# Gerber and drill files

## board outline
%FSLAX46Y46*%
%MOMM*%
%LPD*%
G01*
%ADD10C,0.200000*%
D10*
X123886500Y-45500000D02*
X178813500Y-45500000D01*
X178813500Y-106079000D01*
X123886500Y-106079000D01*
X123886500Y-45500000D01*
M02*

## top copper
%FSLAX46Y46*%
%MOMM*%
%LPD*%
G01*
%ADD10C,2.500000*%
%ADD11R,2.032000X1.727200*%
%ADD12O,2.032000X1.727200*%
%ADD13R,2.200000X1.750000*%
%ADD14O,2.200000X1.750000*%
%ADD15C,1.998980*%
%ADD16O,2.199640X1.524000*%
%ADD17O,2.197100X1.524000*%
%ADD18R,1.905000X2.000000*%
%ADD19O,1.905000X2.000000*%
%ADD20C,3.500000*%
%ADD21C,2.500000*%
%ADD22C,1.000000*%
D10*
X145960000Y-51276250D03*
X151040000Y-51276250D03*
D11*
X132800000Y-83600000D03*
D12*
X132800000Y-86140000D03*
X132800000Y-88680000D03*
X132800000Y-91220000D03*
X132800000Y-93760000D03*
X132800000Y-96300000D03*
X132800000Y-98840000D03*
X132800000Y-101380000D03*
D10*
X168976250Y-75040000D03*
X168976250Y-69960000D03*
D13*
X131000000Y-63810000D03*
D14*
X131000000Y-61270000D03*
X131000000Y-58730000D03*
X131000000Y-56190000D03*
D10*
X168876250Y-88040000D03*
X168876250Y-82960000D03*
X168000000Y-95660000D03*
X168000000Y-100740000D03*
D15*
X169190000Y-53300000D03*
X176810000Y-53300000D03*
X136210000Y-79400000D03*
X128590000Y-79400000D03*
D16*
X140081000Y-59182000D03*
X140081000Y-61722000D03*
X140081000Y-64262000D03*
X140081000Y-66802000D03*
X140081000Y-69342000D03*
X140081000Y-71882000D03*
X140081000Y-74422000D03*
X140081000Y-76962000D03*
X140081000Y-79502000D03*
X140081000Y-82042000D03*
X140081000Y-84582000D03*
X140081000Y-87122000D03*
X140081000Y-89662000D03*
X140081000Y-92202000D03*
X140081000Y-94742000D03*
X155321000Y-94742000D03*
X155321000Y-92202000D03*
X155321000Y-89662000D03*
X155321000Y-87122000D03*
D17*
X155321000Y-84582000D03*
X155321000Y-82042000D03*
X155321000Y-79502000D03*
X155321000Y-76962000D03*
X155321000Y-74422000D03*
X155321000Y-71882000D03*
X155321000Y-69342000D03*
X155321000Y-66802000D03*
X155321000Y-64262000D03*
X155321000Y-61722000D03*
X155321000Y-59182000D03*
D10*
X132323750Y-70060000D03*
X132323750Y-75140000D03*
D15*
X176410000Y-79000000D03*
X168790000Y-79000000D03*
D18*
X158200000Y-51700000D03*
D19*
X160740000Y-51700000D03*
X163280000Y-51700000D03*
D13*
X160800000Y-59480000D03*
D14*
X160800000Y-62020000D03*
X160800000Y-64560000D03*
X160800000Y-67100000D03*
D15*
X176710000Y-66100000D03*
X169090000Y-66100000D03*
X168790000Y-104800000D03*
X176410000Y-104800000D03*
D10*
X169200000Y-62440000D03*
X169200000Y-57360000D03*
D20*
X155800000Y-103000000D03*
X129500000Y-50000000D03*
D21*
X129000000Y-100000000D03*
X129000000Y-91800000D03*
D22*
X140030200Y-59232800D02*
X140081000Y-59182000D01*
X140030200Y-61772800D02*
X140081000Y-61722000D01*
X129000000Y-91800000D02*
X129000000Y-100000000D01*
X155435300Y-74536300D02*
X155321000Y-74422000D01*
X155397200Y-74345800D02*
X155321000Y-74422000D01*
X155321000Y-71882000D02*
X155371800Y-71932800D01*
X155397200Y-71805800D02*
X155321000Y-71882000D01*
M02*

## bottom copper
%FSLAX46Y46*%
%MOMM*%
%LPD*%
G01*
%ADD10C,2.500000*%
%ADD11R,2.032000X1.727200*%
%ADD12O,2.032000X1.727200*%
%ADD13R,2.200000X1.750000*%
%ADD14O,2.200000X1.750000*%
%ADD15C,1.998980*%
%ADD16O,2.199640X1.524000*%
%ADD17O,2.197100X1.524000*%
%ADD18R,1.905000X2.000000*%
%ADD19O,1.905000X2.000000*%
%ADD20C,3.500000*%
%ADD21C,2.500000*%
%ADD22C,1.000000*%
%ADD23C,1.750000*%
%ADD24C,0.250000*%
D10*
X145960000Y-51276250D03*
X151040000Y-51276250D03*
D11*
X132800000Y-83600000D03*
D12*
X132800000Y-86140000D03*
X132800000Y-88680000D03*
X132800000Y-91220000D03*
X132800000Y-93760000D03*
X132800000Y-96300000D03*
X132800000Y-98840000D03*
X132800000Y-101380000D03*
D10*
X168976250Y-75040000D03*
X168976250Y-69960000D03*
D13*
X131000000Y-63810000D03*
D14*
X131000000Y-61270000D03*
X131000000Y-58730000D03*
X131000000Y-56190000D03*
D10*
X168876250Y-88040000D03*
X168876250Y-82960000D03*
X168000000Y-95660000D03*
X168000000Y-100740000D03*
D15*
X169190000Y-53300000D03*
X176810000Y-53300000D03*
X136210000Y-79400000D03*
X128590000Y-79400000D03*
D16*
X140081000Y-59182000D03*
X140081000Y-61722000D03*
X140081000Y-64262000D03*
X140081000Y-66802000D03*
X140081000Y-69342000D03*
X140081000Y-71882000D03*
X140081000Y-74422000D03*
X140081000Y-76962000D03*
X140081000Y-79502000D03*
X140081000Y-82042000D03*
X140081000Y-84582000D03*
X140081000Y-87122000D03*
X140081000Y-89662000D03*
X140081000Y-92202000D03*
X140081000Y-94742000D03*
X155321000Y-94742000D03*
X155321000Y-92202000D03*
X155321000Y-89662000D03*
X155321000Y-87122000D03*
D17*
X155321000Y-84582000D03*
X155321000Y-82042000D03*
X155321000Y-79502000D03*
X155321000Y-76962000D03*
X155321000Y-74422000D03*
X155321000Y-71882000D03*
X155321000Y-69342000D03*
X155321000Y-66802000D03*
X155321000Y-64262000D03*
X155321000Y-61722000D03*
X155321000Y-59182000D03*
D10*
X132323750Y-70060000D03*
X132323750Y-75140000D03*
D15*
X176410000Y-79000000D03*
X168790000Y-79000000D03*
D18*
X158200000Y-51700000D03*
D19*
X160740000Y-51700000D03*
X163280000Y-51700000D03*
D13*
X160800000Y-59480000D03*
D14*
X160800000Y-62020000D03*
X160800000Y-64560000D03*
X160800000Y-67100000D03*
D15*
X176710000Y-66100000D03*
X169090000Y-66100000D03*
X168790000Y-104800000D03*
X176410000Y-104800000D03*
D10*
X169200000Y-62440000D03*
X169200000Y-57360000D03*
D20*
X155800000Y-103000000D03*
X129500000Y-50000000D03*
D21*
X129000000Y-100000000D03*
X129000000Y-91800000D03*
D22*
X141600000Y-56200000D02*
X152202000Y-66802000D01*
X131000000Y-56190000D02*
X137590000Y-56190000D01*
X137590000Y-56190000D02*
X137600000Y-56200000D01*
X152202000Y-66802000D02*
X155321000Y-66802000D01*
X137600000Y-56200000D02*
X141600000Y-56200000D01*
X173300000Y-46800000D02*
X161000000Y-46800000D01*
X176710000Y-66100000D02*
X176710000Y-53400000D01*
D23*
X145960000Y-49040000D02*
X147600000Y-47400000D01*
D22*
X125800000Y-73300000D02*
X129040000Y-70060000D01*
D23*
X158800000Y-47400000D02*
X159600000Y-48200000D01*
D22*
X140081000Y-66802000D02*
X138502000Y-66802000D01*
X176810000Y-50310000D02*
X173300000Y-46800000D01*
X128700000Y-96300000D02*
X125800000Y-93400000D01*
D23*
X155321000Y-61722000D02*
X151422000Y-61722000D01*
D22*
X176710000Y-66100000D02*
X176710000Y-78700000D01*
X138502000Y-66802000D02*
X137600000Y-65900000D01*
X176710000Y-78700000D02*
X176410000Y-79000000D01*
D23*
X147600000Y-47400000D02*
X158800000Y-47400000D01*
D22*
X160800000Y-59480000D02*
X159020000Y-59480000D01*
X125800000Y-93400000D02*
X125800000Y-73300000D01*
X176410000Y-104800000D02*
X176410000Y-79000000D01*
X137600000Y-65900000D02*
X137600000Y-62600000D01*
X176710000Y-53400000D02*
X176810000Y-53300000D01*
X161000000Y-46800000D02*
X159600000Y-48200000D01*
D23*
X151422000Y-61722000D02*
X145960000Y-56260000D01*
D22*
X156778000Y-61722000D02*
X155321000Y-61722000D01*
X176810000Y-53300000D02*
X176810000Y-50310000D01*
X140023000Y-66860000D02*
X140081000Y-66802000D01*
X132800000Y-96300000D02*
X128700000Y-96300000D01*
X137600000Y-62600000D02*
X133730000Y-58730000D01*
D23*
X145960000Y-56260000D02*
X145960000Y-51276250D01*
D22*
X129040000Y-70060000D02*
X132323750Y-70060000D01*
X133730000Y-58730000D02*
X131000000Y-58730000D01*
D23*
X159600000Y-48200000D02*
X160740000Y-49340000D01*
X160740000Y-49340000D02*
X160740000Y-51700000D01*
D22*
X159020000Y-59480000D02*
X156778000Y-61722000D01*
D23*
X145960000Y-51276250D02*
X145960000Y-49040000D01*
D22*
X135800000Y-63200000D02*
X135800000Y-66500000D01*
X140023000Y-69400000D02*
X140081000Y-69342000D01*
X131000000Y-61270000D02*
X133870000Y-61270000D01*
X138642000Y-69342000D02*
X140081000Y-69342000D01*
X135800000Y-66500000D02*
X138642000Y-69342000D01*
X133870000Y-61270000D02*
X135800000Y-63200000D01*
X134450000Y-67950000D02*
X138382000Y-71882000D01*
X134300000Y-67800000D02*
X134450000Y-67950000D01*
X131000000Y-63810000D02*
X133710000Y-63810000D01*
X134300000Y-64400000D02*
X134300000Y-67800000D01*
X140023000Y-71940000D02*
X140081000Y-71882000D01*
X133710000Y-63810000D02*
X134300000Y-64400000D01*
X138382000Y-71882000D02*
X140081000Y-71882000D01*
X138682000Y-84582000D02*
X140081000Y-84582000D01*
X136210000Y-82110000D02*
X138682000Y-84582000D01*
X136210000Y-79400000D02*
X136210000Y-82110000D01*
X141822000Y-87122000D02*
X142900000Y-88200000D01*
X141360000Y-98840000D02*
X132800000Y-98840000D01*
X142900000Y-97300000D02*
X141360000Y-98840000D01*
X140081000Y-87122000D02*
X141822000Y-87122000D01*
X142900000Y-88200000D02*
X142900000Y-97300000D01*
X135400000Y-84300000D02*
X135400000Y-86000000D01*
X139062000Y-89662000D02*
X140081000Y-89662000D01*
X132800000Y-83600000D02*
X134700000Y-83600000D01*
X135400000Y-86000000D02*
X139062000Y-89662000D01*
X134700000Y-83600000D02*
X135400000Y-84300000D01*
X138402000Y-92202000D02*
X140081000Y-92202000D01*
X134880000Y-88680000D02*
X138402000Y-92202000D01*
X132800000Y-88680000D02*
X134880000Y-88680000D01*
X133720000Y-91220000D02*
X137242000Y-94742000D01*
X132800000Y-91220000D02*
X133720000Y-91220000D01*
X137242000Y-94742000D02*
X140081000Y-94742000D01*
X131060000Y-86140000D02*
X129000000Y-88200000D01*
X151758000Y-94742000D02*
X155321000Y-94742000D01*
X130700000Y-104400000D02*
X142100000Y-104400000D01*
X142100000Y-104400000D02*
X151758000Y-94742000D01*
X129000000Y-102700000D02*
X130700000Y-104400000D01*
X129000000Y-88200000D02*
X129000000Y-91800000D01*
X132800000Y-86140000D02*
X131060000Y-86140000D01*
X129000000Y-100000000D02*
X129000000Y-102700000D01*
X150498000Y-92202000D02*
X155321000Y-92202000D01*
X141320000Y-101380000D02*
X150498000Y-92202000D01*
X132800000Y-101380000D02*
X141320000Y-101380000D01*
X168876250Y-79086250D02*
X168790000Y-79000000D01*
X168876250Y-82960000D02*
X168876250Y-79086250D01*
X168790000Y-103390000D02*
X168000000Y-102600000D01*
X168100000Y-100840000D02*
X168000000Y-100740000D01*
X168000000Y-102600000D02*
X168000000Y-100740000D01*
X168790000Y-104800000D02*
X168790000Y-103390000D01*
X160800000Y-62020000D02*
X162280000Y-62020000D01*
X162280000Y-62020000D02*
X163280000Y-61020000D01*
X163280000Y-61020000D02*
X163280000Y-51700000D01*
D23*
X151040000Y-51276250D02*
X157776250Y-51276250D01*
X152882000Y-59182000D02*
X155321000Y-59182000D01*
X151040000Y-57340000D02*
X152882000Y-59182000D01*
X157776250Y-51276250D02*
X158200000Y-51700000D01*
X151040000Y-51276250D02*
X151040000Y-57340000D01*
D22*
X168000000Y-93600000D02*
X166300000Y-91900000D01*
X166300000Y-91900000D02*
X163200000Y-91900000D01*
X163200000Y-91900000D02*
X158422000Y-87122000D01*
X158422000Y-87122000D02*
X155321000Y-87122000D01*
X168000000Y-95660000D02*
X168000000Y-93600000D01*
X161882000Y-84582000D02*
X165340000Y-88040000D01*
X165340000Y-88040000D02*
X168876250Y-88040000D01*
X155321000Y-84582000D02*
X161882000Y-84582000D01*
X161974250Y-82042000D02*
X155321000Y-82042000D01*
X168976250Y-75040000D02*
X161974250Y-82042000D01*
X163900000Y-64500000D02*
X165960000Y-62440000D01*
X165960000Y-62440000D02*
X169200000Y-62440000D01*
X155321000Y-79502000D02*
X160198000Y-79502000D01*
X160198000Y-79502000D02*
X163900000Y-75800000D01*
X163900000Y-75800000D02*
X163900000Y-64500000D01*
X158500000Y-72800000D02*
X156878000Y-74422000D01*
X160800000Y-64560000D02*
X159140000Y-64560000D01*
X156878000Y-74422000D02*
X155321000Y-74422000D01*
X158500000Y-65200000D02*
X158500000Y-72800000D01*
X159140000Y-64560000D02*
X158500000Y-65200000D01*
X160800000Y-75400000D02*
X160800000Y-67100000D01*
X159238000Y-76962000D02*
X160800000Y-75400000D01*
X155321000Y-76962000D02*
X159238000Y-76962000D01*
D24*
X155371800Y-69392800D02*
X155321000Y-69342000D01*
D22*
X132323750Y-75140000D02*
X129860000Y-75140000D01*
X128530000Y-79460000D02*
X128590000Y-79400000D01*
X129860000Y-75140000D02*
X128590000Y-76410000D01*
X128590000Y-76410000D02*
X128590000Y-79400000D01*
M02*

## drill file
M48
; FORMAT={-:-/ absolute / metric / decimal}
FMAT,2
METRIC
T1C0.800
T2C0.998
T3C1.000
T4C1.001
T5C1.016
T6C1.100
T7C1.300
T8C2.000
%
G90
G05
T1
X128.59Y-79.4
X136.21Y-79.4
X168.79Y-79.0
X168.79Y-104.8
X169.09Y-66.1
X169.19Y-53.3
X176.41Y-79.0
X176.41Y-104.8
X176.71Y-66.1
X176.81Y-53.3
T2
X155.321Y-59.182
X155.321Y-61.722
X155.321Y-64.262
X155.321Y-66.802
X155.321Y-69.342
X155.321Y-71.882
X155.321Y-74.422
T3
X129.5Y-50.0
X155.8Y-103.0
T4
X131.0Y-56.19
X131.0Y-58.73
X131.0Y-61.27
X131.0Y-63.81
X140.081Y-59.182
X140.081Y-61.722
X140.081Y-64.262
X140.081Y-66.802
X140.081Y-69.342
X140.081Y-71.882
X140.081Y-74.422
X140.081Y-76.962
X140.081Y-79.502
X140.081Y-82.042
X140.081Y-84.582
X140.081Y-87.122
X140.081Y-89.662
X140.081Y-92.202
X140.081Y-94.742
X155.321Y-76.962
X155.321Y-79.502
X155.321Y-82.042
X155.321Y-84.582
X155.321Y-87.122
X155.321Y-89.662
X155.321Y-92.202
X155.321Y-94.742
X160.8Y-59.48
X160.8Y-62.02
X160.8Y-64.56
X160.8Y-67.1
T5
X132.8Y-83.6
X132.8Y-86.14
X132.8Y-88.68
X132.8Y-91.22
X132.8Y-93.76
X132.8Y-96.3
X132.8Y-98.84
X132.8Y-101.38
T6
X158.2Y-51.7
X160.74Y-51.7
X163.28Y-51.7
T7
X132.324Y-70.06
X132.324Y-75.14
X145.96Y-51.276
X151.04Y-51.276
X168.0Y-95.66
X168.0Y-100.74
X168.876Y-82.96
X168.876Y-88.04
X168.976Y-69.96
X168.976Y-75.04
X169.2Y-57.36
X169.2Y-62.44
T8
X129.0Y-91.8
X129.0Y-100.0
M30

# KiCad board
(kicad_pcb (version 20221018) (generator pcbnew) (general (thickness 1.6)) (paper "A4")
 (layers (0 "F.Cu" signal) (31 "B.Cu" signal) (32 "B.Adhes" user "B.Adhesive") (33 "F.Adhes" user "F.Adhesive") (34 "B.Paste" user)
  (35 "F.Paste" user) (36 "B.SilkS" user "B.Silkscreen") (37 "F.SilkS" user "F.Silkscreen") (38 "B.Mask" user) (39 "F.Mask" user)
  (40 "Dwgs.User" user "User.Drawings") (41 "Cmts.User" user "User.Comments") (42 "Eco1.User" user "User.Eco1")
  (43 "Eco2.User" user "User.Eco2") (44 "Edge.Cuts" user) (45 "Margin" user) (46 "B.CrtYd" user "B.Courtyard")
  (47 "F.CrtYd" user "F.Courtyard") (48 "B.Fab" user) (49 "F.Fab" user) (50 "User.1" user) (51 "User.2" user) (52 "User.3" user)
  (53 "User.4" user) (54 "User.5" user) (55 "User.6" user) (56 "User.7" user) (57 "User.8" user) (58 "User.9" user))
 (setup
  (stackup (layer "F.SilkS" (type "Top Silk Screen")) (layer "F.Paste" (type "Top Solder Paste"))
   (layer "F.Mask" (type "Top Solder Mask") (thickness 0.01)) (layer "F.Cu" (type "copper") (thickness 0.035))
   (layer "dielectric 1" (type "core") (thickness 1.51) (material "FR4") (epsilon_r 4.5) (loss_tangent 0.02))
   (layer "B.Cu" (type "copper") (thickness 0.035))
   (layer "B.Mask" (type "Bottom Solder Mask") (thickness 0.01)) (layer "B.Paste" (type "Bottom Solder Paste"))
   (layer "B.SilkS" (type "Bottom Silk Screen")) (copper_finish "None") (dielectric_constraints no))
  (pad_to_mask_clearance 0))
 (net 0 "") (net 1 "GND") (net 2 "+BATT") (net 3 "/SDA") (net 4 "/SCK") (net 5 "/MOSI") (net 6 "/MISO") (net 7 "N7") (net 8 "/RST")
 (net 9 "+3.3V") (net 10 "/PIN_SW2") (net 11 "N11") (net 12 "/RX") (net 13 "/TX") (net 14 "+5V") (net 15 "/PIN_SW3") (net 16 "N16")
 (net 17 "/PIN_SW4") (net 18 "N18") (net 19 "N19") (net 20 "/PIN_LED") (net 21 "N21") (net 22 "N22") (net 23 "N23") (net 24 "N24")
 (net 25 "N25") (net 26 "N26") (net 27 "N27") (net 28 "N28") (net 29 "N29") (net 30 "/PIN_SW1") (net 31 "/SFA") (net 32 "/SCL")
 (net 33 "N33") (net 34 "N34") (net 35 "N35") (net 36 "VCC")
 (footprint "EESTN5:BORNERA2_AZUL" (layer "F.Cu") (at 148.5 51.27625)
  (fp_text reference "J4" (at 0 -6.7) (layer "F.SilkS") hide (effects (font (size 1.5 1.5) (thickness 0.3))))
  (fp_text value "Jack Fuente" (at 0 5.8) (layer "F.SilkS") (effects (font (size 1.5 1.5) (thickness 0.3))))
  (pad "1" thru_hole circle (at -2.54 0) (size 2.5 2.5) (drill 1.3) (layers "*.Cu" "*.Mask" "F.SilkS") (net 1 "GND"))
  (pad "2" thru_hole circle (at 2.54 0) (size 2.5 2.5) (drill 1.3) (layers "*.Cu" "*.Mask" "F.SilkS") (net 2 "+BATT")))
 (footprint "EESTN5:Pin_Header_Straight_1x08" (layer "F.Cu") (at 132.8 83.6)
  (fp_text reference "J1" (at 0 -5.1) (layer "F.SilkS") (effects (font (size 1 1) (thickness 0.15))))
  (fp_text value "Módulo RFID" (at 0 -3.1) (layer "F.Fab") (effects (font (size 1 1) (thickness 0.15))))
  (pad "1" thru_hole rect (at 0 0) (size 2.032 1.7272) (drill 1.016) (layers "*.Cu" "*.Mask" "F.SilkS") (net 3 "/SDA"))
  (pad "2" thru_hole oval (at 0 2.54) (size 2.032 1.7272) (drill 1.016) (layers "*.Cu" "*.Mask" "F.SilkS") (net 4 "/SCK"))
  (pad "3" thru_hole oval (at 0 5.08) (size 2.032 1.7272) (drill 1.016) (layers "*.Cu" "*.Mask" "F.SilkS") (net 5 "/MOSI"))
  (pad "4" thru_hole oval (at 0 7.62) (size 2.032 1.7272) (drill 1.016) (layers "*.Cu" "*.Mask" "F.SilkS") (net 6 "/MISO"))
  (pad "5" thru_hole oval (at 0 10.16) (size 2.032 1.7272) (drill 1.016) (layers "*.Cu" "*.Mask" "F.SilkS") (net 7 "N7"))
  (pad "6" thru_hole oval (at 0 12.7) (size 2.032 1.7272) (drill 1.016) (layers "*.Cu" "*.Mask" "F.SilkS") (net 1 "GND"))
  (pad "7" thru_hole oval (at 0 15.24) (size 2.032 1.7272) (drill 1.016) (layers "*.Cu" "*.Mask" "F.SilkS") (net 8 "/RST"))
  (pad "8" thru_hole oval (at 0 17.78) (size 2.032 1.7272) (drill 1.016) (layers "*.Cu" "*.Mask" "F.SilkS") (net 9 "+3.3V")))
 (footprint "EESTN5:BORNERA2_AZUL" (layer "F.Cu") (at 168.97625 72.5 90)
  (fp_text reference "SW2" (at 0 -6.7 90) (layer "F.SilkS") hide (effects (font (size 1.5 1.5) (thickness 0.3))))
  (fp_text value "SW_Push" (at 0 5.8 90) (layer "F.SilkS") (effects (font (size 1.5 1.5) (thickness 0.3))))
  (pad "1" thru_hole circle (at -2.54 0 90) (size 2.5 2.5) (drill 1.3) (layers "*.Cu" "*.Mask" "F.SilkS") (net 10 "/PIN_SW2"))
  (pad "2" thru_hole circle (at 2.54 0 90) (size 2.5 2.5) (drill 1.3) (layers "*.Cu" "*.Mask" "F.SilkS") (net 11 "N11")))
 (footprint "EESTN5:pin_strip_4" (layer "F.Cu") (at 131 60 90)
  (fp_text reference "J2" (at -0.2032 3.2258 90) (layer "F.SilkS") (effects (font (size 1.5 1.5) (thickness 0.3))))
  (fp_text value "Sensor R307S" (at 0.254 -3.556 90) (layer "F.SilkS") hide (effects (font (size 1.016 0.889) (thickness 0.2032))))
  (pad "1" thru_hole rect (at -3.81 0 90) (size 1.75 2.2) (drill 1.00076) (layers "*.Cu" "*.Mask" "F.SilkS") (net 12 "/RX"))
  (pad "2" thru_hole oval (at -1.27 0 90) (size 1.75 2.2) (drill 1.00076) (layers "*.Cu" "*.Mask" "F.SilkS") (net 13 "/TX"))
  (pad "3" thru_hole oval (at 1.27 0 90) (size 1.75 2.2) (drill 1.00076) (layers "*.Cu" "*.Mask" "F.SilkS") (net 1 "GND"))
  (pad "4" thru_hole oval (at 3.81 0 90) (size 1.75 2.2) (drill 1.00076) (layers "*.Cu" "*.Mask" "F.SilkS") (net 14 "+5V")))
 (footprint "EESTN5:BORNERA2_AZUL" (layer "F.Cu") (at 168.87625 85.5 90)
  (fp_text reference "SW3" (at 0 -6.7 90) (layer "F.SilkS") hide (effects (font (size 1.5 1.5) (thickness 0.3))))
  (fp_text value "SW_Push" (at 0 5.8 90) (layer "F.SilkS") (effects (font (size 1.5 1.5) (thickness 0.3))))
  (pad "1" thru_hole circle (at -2.54 0 90) (size 2.5 2.5) (drill 1.3) (layers "*.Cu" "*.Mask" "F.SilkS") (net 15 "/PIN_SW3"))
  (pad "2" thru_hole circle (at 2.54 0 90) (size 2.5 2.5) (drill 1.3) (layers "*.Cu" "*.Mask" "F.SilkS") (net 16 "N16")))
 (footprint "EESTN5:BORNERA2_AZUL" (layer "F.Cu") (at 168 98.2 -90)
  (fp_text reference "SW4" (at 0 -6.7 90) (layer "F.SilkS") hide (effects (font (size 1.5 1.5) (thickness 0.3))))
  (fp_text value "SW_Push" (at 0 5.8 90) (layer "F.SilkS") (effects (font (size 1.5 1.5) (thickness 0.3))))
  (pad "1" thru_hole circle (at -2.54 0 270) (size 2.5 2.5) (drill 1.3) (layers "*.Cu" "*.Mask" "F.SilkS") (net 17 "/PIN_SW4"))
  (pad "2" thru_hole circle (at 2.54 0 270) (size 2.5 2.5) (drill 1.3) (layers "*.Cu" "*.Mask" "F.SilkS") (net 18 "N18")))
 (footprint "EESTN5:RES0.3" (layer "F.Cu") (at 173 53.3)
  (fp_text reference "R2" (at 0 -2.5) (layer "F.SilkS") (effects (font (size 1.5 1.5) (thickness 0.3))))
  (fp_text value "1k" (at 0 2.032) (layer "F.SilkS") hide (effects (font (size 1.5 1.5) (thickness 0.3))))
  (pad "1" thru_hole circle (at -3.81 0) (size 1.99898 1.99898) (drill 0.8001) (layers "*.Cu" "*.Mask" "F.SilkS") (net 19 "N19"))
  (pad "2" thru_hole circle (at 3.81 0) (size 1.99898 1.99898) (drill 0.8001) (layers "*.Cu" "*.Mask" "F.SilkS") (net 1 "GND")))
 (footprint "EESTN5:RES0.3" (layer "F.Cu") (at 132.4 79.4 180)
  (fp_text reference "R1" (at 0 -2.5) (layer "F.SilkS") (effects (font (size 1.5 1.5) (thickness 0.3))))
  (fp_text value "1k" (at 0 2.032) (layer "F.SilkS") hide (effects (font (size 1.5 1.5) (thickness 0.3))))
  (pad "1" thru_hole circle (at -3.81 0 180) (size 1.99898 1.99898) (drill 0.8001) (layers "*.Cu" "*.Mask" "F.SilkS") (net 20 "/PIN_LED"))
  (pad "2" thru_hole circle (at 3.81 0 180) (size 1.99898 1.99898) (drill 0.8001) (layers "*.Cu" "*.Mask" "F.SilkS") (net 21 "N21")))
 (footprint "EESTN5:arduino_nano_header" (layer "F.Cu") (at 147.701 76.962 -90)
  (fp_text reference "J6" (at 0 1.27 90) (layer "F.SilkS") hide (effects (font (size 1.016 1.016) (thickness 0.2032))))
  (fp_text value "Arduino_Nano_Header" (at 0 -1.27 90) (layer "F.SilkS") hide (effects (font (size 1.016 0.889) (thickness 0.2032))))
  (pad "1" thru_hole oval (at -17.78 7.62 270) (size 1.524 2.19964) (drill 1.00076) (layers "*.Cu" "*.Mask" "F.SilkS") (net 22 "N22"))
  (pad "2" thru_hole oval (at -15.24 7.62 270) (size 1.524 2.19964) (drill 1.00076) (layers "*.Cu" "*.Mask" "F.SilkS") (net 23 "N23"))
  (pad "3" thru_hole oval (at -12.7 7.62 270) (size 1.524 2.19964) (drill 1.00076) (layers "*.Cu" "*.Mask" "F.SilkS") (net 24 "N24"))
  (pad "4" thru_hole oval (at -10.16 7.62 270) (size 1.524 2.19964) (drill 1.00076) (layers "*.Cu" "*.Mask" "F.SilkS") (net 1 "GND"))
  (pad "5" thru_hole oval (at -7.62 7.62 270) (size 1.524 2.19964) (drill 1.00076) (layers "*.Cu" "*.Mask" "F.SilkS") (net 13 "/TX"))
  (pad "6" thru_hole oval (at -5.08 7.62 270) (size 1.524 2.19964) (drill 1.00076) (layers "*.Cu" "*.Mask" "F.SilkS") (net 12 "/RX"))
  (pad "7" thru_hole oval (at -2.54 7.62 270) (size 1.524 2.19964) (drill 1.00076) (layers "*.Cu" "*.Mask" "F.SilkS") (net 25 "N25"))
  (pad "8" thru_hole oval (at 0 7.62 270) (size 1.524 2.19964) (drill 1.00076) (layers "*.Cu" "*.Mask" "F.SilkS") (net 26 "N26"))
  (pad "9" thru_hole oval (at 2.54 7.62 270) (size 1.524 2.19964) (drill 1.00076) (layers "*.Cu" "*.Mask" "F.SilkS") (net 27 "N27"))
  (pad "10" thru_hole oval (at 5.08 7.62 270) (size 1.524 2.19964) (drill 1.00076) (layers "*.Cu" "*.Mask" "F.SilkS") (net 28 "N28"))
  (pad "11" thru_hole oval (at 7.62 7.62 270) (size 1.524 2.19964) (drill 1.00076) (layers "*.Cu" "*.Mask" "F.SilkS") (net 20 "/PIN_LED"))
  (pad "12" thru_hole oval (at 10.16 7.62 270) (size 1.524 2.19964) (drill 1.00076) (layers "*.Cu" "*.Mask" "F.SilkS") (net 8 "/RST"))
  (pad "13" thru_hole oval (at 12.7 7.62 270) (size 1.524 2.19964) (drill 1.00076) (layers "*.Cu" "*.Mask" "F.SilkS") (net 3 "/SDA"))
  (pad "14" thru_hole oval (at 15.24 7.62 270) (size 1.524 2.19964) (drill 1.00076) (layers "*.Cu" "*.Mask" "F.SilkS") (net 5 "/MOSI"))
  (pad "15" thru_hole oval (at 17.78 7.62 270) (size 1.524 2.19964) (drill 1.00076) (layers "*.Cu" "*.Mask" "F.SilkS") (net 6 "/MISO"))
  (pad "16" thru_hole oval (at 17.78 -7.62 270) (size 1.524 2.19964) (drill 1.00076) (layers "*.Cu" "*.Mask" "F.SilkS") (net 4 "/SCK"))
  (pad "17" thru_hole oval (at 15.24 -7.62 270) (size 1.524 2.19964) (drill 1.00076) (layers "*.Cu" "*.Mask" "F.SilkS") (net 9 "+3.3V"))
  (pad "18" thru_hole oval (at 12.7 -7.62 270) (size 1.524 2.19964) (drill 1.00076) (layers "*.Cu" "*.Mask" "F.SilkS") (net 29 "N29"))
  (pad "19" thru_hole oval (at 10.16 -7.62 270) (size 1.524 2.19964) (drill 1.00076) (layers "*.Cu" "*.Mask" "F.SilkS") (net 17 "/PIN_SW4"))
  (pad "20" thru_hole oval (at 7.62 -7.62 270) (size 1.524 2.1971) (drill 1.00076) (layers "*.Cu" "*.Mask" "F.SilkS") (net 15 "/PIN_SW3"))
  (pad "21" thru_hole oval (at 5.08 -7.62 270) (size 1.524 2.1971) (drill 1.00076) (layers "*.Cu" "*.Mask" "F.SilkS") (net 10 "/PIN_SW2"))
  (pad "22" thru_hole oval (at 2.54 -7.62 270) (size 1.524 2.1971) (drill 1.00076) (layers "*.Cu" "*.Mask" "F.SilkS") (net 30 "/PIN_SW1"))
  (pad "23" thru_hole oval (at 0 -7.62 270) (size 1.524 2.1971) (drill 1.00076) (layers "*.Cu" "*.Mask" "F.SilkS") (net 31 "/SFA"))
  (pad "24" thru_hole oval (at -2.54 -7.62 270) (size 1.524 2.1971) (drill 0.99822) (layers "*.Cu" "*.Mask" "F.SilkS") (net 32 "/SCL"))
  (pad "25" thru_hole oval (at -5.08 -7.62 270) (size 1.524 2.1971) (drill 0.99822) (layers "*.Cu" "*.Mask" "F.SilkS") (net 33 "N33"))
  (pad "26" thru_hole oval (at -7.62 -7.62 270) (size 1.524 2.1971) (drill 0.99822) (layers "*.Cu" "*.Mask" "F.SilkS") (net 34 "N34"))
  (pad "27" thru_hole oval (at -10.16 -7.62 270) (size 1.524 2.1971) (drill 0.99822) (layers "*.Cu" "*.Mask" "F.SilkS") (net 14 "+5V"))
  (pad "28" thru_hole oval (at -12.7 -7.62 270) (size 1.524 2.1971) (drill 0.99822) (layers "*.Cu" "*.Mask" "F.SilkS") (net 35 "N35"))
  (pad "29" thru_hole oval (at -15.24 -7.62 270) (size 1.524 2.1971) (drill 0.99822) (layers "*.Cu" "*.Mask" "F.SilkS") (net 1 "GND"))
  (pad "30" thru_hole oval (at -17.78 -7.62 270) (size 1.524 2.1971) (drill 0.99822) (layers "*.Cu" "*.Mask" "F.SilkS") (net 2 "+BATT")))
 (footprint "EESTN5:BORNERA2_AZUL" (layer "F.Cu") (at 132.32375 72.6 -90)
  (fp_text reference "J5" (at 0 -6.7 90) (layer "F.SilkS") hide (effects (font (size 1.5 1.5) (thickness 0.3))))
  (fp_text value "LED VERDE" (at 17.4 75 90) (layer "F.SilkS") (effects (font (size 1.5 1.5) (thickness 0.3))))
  (pad "1" thru_hole circle (at -2.54 0 270) (size 2.5 2.5) (drill 1.3) (layers "*.Cu" "*.Mask" "F.SilkS") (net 1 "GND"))
  (pad "2" thru_hole circle (at 2.54 0 270) (size 2.5 2.5) (drill 1.3) (layers "*.Cu" "*.Mask" "F.SilkS") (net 21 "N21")))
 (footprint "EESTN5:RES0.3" (layer "F.Cu") (at 172.6 79 180)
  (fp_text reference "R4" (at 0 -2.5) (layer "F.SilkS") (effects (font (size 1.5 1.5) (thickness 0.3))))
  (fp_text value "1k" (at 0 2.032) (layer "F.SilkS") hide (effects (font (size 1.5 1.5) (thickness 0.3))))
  (pad "1" thru_hole circle (at -3.81 0 180) (size 1.99898 1.99898) (drill 0.8001) (layers "*.Cu" "*.Mask" "F.SilkS") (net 1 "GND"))
  (pad "2" thru_hole circle (at 3.81 0 180) (size 1.99898 1.99898) (drill 0.8001) (layers "*.Cu" "*.Mask" "F.SilkS") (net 16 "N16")))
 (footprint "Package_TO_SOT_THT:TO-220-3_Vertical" (layer "F.Cu") (at 158.2 51.7)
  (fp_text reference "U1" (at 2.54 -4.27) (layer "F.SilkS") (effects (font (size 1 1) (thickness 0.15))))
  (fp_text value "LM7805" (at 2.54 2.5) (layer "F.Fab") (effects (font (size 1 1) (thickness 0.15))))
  (pad "1" thru_hole rect (at 0 0) (size 1.905 2) (drill 1.1) (layers "*.Cu" "*.Mask") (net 2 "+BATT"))
  (pad "2" thru_hole oval (at 2.54 0) (size 1.905 2) (drill 1.1) (layers "*.Cu" "*.Mask") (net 1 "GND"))
  (pad "3" thru_hole oval (at 5.08 0) (size 1.905 2) (drill 1.1) (layers "*.Cu" "*.Mask") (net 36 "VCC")))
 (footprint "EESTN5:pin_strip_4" (layer "F.Cu") (at 160.8 63.29 -90)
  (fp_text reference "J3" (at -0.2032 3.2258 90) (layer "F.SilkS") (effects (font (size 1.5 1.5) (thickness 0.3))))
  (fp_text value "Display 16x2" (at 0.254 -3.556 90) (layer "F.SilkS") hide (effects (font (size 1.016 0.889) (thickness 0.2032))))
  (pad "1" thru_hole rect (at -3.81 0 270) (size 1.75 2.2) (drill 1.00076) (layers "*.Cu" "*.Mask" "F.SilkS") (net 1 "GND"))
  (pad "2" thru_hole oval (at -1.27 0 270) (size 1.75 2.2) (drill 1.00076) (layers "*.Cu" "*.Mask" "F.SilkS") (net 36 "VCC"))
  (pad "3" thru_hole oval (at 1.27 0 270) (size 1.75 2.2) (drill 1.00076) (layers "*.Cu" "*.Mask" "F.SilkS") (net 32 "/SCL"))
  (pad "4" thru_hole oval (at 3.81 0 270) (size 1.75 2.2) (drill 1.00076) (layers "*.Cu" "*.Mask" "F.SilkS") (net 31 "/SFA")))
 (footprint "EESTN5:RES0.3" (layer "F.Cu") (at 172.9 66.1 180)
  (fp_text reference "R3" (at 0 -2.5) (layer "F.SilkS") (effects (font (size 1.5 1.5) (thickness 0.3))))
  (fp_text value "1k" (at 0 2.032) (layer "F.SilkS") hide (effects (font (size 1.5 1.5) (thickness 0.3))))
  (pad "1" thru_hole circle (at -3.81 0 180) (size 1.99898 1.99898) (drill 0.8001) (layers "*.Cu" "*.Mask" "F.SilkS") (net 1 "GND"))
  (pad "2" thru_hole circle (at 3.81 0 180) (size 1.99898 1.99898) (drill 0.8001) (layers "*.Cu" "*.Mask" "F.SilkS") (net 11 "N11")))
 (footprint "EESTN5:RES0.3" (layer "F.Cu") (at 172.6 104.8)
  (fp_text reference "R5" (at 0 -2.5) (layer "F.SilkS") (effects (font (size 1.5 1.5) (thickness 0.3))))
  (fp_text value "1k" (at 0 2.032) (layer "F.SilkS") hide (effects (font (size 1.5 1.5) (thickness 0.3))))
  (pad "1" thru_hole circle (at -3.81 0) (size 1.99898 1.99898) (drill 0.8001) (layers "*.Cu" "*.Mask" "F.SilkS") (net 18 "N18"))
  (pad "2" thru_hole circle (at 3.81 0) (size 1.99898 1.99898) (drill 0.8001) (layers "*.Cu" "*.Mask" "F.SilkS") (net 1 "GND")))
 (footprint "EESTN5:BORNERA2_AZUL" (layer "F.Cu") (at 169.2 59.9 90)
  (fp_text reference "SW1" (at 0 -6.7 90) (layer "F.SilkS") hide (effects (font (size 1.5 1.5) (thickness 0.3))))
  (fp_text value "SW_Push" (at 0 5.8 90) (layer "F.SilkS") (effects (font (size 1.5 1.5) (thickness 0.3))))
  (pad "1" thru_hole circle (at -2.54 0 90) (size 2.5 2.5) (drill 1.3) (layers "*.Cu" "*.Mask" "F.SilkS") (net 30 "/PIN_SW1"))
  (pad "2" thru_hole circle (at 2.54 0 90) (size 2.5 2.5) (drill 1.3) (layers "*.Cu" "*.Mask" "F.SilkS") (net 19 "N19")))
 (gr_rect (start 123.8865 45.5) (end 178.8135 106.079) (stroke (width 0.2) (type default)) (fill none) (layer "Edge.Cuts"))
 (via (at 155.8 103) (size 3.5) (drill 1) (layers "F.Cu" "B.Cu") (free) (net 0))
 (via (at 129.5 50) (size 3.5) (drill 1) (layers "F.Cu" "B.Cu") (free) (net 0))
 (segment (start 141.6 56.2) (end 152.202 66.802) (width 1) (layer "B.Cu") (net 14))
 (segment (start 131 56.19) (end 137.59 56.19) (width 1) (layer "B.Cu") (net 14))
 (segment (start 137.59 56.19) (end 137.6 56.2) (width 1) (layer "B.Cu") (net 14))
 (segment (start 152.202 66.802) (end 155.321 66.802) (width 1) (layer "B.Cu") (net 14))
 (segment (start 137.6 56.2) (end 141.6 56.2) (width 1) (layer "B.Cu") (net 14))
 (segment (start 173.3 46.8) (end 161 46.8) (width 1) (layer "B.Cu") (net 1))
 (segment (start 176.71 66.1) (end 176.71 53.4) (width 1) (layer "B.Cu") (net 1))
 (segment (start 145.96 49.04) (end 147.6 47.4) (width 1.75) (layer "B.Cu") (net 1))
 (segment (start 125.8 73.3) (end 129.04 70.06) (width 1) (layer "B.Cu") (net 1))
 (segment (start 158.8 47.4) (end 159.6 48.2) (width 1.75) (layer "B.Cu") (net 1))
 (segment (start 140.081 66.802) (end 138.502 66.802) (width 1) (layer "B.Cu") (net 1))
 (segment (start 176.81 50.31) (end 173.3 46.8) (width 1) (layer "B.Cu") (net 1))
 (segment (start 128.7 96.3) (end 125.8 93.4) (width 1) (layer "B.Cu") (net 1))
 (segment (start 155.321 61.722) (end 151.422 61.722) (width 1.75) (layer "B.Cu") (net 1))
 (segment (start 176.71 66.1) (end 176.71 78.7) (width 1) (layer "B.Cu") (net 1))
 (segment (start 138.502 66.802) (end 137.6 65.9) (width 1) (layer "B.Cu") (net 1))
 (segment (start 176.71 78.7) (end 176.41 79) (width 1) (layer "B.Cu") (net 1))
 (segment (start 147.6 47.4) (end 158.8 47.4) (width 1.75) (layer "B.Cu") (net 1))
 (segment (start 160.8 59.48) (end 159.02 59.48) (width 1) (layer "B.Cu") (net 1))
 (segment (start 125.8 93.4) (end 125.8 73.3) (width 1) (layer "B.Cu") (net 1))
 (segment (start 176.41 104.8) (end 176.41 79) (width 1) (layer "B.Cu") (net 1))
 (segment (start 137.6 65.9) (end 137.6 62.6) (width 1) (layer "B.Cu") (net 1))
 (segment (start 176.71 53.4) (end 176.81 53.3) (width 1) (layer "B.Cu") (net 1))
 (segment (start 161 46.8) (end 159.6 48.2) (width 1) (layer "B.Cu") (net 1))
 (segment (start 151.422 61.722) (end 145.96 56.26) (width 1.75) (layer "B.Cu") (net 1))
 (segment (start 156.778 61.722) (end 155.321 61.722) (width 1) (layer "B.Cu") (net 1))
 (segment (start 176.81 53.3) (end 176.81 50.31) (width 1) (layer "B.Cu") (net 1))
 (segment (start 140.023 66.86) (end 140.081 66.802) (width 1) (layer "B.Cu") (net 1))
 (segment (start 132.8 96.3) (end 128.7 96.3) (width 1) (layer "B.Cu") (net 1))
 (segment (start 137.6 62.6) (end 133.73 58.73) (width 1) (layer "B.Cu") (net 1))
 (segment (start 145.96 56.26) (end 145.96 51.27625) (width 1.75) (layer "B.Cu") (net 1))
 (segment (start 129.04 70.06) (end 132.32375 70.06) (width 1) (layer "B.Cu") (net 1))
 (segment (start 133.73 58.73) (end 131 58.73) (width 1) (layer "B.Cu") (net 1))
 (segment (start 159.6 48.2) (end 160.74 49.34) (width 1.75) (layer "B.Cu") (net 1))
 (segment (start 160.74 49.34) (end 160.74 51.7) (width 1.75) (layer "B.Cu") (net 1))
 (segment (start 159.02 59.48) (end 156.778 61.722) (width 1) (layer "B.Cu") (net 1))
 (segment (start 145.96 51.27625) (end 145.96 49.04) (width 1.75) (layer "B.Cu") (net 1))
 (segment (start 140.0302 59.2328) (end 140.081 59.182) (width 1) (layer "F.Cu") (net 22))
 (segment (start 140.0302 61.7728) (end 140.081 61.722) (width 1) (layer "F.Cu") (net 23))
 (segment (start 135.8 63.2) (end 135.8 66.5) (width 1) (layer "B.Cu") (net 13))
 (segment (start 140.023 69.4) (end 140.081 69.342) (width 1) (layer "B.Cu") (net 13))
 (segment (start 131 61.27) (end 133.87 61.27) (width 1) (layer "B.Cu") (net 13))
 (segment (start 138.642 69.342) (end 140.081 69.342) (width 1) (layer "B.Cu") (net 13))
 (segment (start 135.8 66.5) (end 138.642 69.342) (width 1) (layer "B.Cu") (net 13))
 (segment (start 133.87 61.27) (end 135.8 63.2) (width 1) (layer "B.Cu") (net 13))
 (segment (start 134.45 67.95) (end 138.382 71.882) (width 1) (layer "B.Cu") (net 12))
 (segment (start 134.3 67.8) (end 134.45 67.95) (width 1) (layer "B.Cu") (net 12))
 (segment (start 131 63.81) (end 133.71 63.81) (width 1) (layer "B.Cu") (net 12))
 (segment (start 134.3 64.4) (end 134.3 67.8) (width 1) (layer "B.Cu") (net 12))
 (segment (start 140.023 71.94) (end 140.081 71.882) (width 1) (layer "B.Cu") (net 12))
 (segment (start 133.71 63.81) (end 134.3 64.4) (width 1) (layer "B.Cu") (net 12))
 (segment (start 138.382 71.882) (end 140.081 71.882) (width 1) (layer "B.Cu") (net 12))
 (segment (start 138.682 84.582) (end 140.081 84.582) (width 1) (layer "B.Cu") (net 20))
 (segment (start 136.21 82.11) (end 138.682 84.582) (width 1) (layer "B.Cu") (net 20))
 (segment (start 136.21 79.4) (end 136.21 82.11) (width 1) (layer "B.Cu") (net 20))
 (segment (start 141.822 87.122) (end 142.9 88.2) (width 1) (layer "B.Cu") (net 8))
 (segment (start 141.36 98.84) (end 132.8 98.84) (width 1) (layer "B.Cu") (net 8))
 (segment (start 142.9 97.3) (end 141.36 98.84) (width 1) (layer "B.Cu") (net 8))
 (segment (start 140.081 87.122) (end 141.822 87.122) (width 1) (layer "B.Cu") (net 8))
 (segment (start 142.9 88.2) (end 142.9 97.3) (width 1) (layer "B.Cu") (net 8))
 (segment (start 135.4 84.3) (end 135.4 86) (width 1) (layer "B.Cu") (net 3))
 (segment (start 139.062 89.662) (end 140.081 89.662) (width 1) (layer "B.Cu") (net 3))
 (segment (start 132.8 83.6) (end 134.7 83.6) (width 1) (layer "B.Cu") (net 3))
 (segment (start 135.4 86) (end 139.062 89.662) (width 1) (layer "B.Cu") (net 3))
 (segment (start 134.7 83.6) (end 135.4 84.3) (width 1) (layer "B.Cu") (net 3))
 (segment (start 138.402 92.202) (end 140.081 92.202) (width 1) (layer "B.Cu") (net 5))
 (segment (start 134.88 88.68) (end 138.402 92.202) (width 1) (layer "B.Cu") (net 5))
 (segment (start 132.8 88.68) (end 134.88 88.68) (width 1) (layer "B.Cu") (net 5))
 (segment (start 133.72 91.22) (end 137.242 94.742) (width 1) (layer "B.Cu") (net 6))
 (segment (start 132.8 91.22) (end 133.72 91.22) (width 1) (layer "B.Cu") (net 6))
 (segment (start 137.242 94.742) (end 140.081 94.742) (width 1) (layer "B.Cu") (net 6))
 (segment (start 129 91.8) (end 129 100) (width 1) (layer "F.Cu") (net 4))
 (via (at 129 100) (size 2.5) (drill 2) (layers "F.Cu" "B.Cu") (free) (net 4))
 (via (at 129 91.8) (size 2.5) (drill 2) (layers "F.Cu" "B.Cu") (free) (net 4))
 (segment (start 131.06 86.14) (end 129 88.2) (width 1) (layer "B.Cu") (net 4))
 (segment (start 151.758 94.742) (end 155.321 94.742) (width 1) (layer "B.Cu") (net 4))
 (segment (start 130.7 104.4) (end 142.1 104.4) (width 1) (layer "B.Cu") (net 4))
 (segment (start 142.1 104.4) (end 151.758 94.742) (width 1) (layer "B.Cu") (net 4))
 (segment (start 129 102.7) (end 130.7 104.4) (width 1) (layer "B.Cu") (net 4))
 (segment (start 129 88.2) (end 129 91.8) (width 1) (layer "B.Cu") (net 4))
 (segment (start 132.8 86.14) (end 131.06 86.14) (width 1) (layer "B.Cu") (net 4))
 (segment (start 129 100) (end 129 102.7) (width 1) (layer "B.Cu") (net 4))
 (segment (start 150.498 92.202) (end 155.321 92.202) (width 1) (layer "B.Cu") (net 9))
 (segment (start 141.32 101.38) (end 150.498 92.202) (width 1) (layer "B.Cu") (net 9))
 (segment (start 132.8 101.38) (end 141.32 101.38) (width 1) (layer "B.Cu") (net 9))
 (segment (start 168.87625 79.08625) (end 168.79 79) (width 1) (layer "B.Cu") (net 16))
 (segment (start 168.87625 82.96) (end 168.87625 79.08625) (width 1) (layer "B.Cu") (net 16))
 (segment (start 168.79 103.39) (end 168 102.6) (width 1) (layer "B.Cu") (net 18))
 (segment (start 168.1 100.84) (end 168 100.74) (width 1) (layer "B.Cu") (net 18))
 (segment (start 168 102.6) (end 168 100.74) (width 1) (layer "B.Cu") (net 18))
 (segment (start 168.79 104.8) (end 168.79 103.39) (width 1) (layer "B.Cu") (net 18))
 (segment (start 160.8 62.02) (end 162.28 62.02) (width 1) (layer "B.Cu") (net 36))
 (segment (start 162.28 62.02) (end 163.28 61.02) (width 1) (layer "B.Cu") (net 36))
 (segment (start 163.28 61.02) (end 163.28 51.7) (width 1) (layer "B.Cu") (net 36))
 (segment (start 151.04 51.27625) (end 157.77625 51.27625) (width 1.75) (layer "B.Cu") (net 2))
 (segment (start 152.882 59.182) (end 155.321 59.182) (width 1.75) (layer "B.Cu") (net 2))
 (segment (start 151.04 57.34) (end 152.882 59.182) (width 1.75) (layer "B.Cu") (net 2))
 (segment (start 157.77625 51.27625) (end 158.2 51.7) (width 1.75) (layer "B.Cu") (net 2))
 (segment (start 151.04 51.27625) (end 151.04 57.34) (width 1.75) (layer "B.Cu") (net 2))
 (segment (start 168 93.6) (end 166.3 91.9) (width 1) (layer "B.Cu") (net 17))
 (segment (start 166.3 91.9) (end 163.2 91.9) (width 1) (layer "B.Cu") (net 17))
 (segment (start 163.2 91.9) (end 158.422 87.122) (width 1) (layer "B.Cu") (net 17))
 (segment (start 158.422 87.122) (end 155.321 87.122) (width 1) (layer "B.Cu") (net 17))
 (segment (start 168 95.66) (end 168 93.6) (width 1) (layer "B.Cu") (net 17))
 (segment (start 161.882 84.582) (end 165.34 88.04) (width 1) (layer "B.Cu") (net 15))
 (segment (start 165.34 88.04) (end 168.87625 88.04) (width 1) (layer "B.Cu") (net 15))
 (segment (start 155.321 84.582) (end 161.882 84.582) (width 1) (layer "B.Cu") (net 15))
 (segment (start 161.97425 82.042) (end 155.321 82.042) (width 1) (layer "B.Cu") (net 10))
 (segment (start 168.97625 75.04) (end 161.97425 82.042) (width 1) (layer "B.Cu") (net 10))
 (segment (start 163.9 64.5) (end 165.96 62.44) (width 1) (layer "B.Cu") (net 30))
 (segment (start 165.96 62.44) (end 169.2 62.44) (width 1) (layer "B.Cu") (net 30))
 (segment (start 155.321 79.502) (end 160.198 79.502) (width 1) (layer "B.Cu") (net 30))
 (segment (start 160.198 79.502) (end 163.9 75.8) (width 1) (layer "B.Cu") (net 30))
 (segment (start 163.9 75.8) (end 163.9 64.5) (width 1) (layer "B.Cu") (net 30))
 (segment (start 155.4353 74.5363) (end 155.321 74.422) (width 1) (layer "F.Cu") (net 32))
 (segment (start 155.3972 74.3458) (end 155.321 74.422) (width 1) (layer "F.Cu") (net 32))
 (segment (start 158.5 72.8) (end 156.878 74.422) (width 1) (layer "B.Cu") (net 32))
 (segment (start 160.8 64.56) (end 159.14 64.56) (width 1) (layer "B.Cu") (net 32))
 (segment (start 156.878 74.422) (end 155.321 74.422) (width 1) (layer "B.Cu") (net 32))
 (segment (start 158.5 65.2) (end 158.5 72.8) (width 1) (layer "B.Cu") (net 32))
 (segment (start 159.14 64.56) (end 158.5 65.2) (width 1) (layer "B.Cu") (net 32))
 (segment (start 160.8 75.4) (end 160.8 67.1) (width 1) (layer "B.Cu") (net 31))
 (segment (start 159.238 76.962) (end 160.8 75.4) (width 1) (layer "B.Cu") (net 31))
 (segment (start 155.321 76.962) (end 159.238 76.962) (width 1) (layer "B.Cu") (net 31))
 (segment (start 155.321 71.882) (end 155.3718 71.9328) (width 1) (layer "F.Cu") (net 33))
 (segment (start 155.3972 71.8058) (end 155.321 71.882) (width 1) (layer "F.Cu") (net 33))
 (segment (start 155.3718 69.3928) (end 155.321 69.342) (width 0.25) (layer "B.Cu") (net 34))
 (segment (start 132.32375 75.14) (end 129.86 75.14) (width 1) (layer "B.Cu") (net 21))
 (segment (start 128.53 79.46) (end 128.59 79.4) (width 1) (layer "B.Cu") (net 21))
 (segment (start 129.86 75.14) (end 128.59 76.41) (width 1) (layer "B.Cu") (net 21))
 (segment (start 128.59 76.41) (end 128.59 79.4) (width 1) (layer "B.Cu") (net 21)))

